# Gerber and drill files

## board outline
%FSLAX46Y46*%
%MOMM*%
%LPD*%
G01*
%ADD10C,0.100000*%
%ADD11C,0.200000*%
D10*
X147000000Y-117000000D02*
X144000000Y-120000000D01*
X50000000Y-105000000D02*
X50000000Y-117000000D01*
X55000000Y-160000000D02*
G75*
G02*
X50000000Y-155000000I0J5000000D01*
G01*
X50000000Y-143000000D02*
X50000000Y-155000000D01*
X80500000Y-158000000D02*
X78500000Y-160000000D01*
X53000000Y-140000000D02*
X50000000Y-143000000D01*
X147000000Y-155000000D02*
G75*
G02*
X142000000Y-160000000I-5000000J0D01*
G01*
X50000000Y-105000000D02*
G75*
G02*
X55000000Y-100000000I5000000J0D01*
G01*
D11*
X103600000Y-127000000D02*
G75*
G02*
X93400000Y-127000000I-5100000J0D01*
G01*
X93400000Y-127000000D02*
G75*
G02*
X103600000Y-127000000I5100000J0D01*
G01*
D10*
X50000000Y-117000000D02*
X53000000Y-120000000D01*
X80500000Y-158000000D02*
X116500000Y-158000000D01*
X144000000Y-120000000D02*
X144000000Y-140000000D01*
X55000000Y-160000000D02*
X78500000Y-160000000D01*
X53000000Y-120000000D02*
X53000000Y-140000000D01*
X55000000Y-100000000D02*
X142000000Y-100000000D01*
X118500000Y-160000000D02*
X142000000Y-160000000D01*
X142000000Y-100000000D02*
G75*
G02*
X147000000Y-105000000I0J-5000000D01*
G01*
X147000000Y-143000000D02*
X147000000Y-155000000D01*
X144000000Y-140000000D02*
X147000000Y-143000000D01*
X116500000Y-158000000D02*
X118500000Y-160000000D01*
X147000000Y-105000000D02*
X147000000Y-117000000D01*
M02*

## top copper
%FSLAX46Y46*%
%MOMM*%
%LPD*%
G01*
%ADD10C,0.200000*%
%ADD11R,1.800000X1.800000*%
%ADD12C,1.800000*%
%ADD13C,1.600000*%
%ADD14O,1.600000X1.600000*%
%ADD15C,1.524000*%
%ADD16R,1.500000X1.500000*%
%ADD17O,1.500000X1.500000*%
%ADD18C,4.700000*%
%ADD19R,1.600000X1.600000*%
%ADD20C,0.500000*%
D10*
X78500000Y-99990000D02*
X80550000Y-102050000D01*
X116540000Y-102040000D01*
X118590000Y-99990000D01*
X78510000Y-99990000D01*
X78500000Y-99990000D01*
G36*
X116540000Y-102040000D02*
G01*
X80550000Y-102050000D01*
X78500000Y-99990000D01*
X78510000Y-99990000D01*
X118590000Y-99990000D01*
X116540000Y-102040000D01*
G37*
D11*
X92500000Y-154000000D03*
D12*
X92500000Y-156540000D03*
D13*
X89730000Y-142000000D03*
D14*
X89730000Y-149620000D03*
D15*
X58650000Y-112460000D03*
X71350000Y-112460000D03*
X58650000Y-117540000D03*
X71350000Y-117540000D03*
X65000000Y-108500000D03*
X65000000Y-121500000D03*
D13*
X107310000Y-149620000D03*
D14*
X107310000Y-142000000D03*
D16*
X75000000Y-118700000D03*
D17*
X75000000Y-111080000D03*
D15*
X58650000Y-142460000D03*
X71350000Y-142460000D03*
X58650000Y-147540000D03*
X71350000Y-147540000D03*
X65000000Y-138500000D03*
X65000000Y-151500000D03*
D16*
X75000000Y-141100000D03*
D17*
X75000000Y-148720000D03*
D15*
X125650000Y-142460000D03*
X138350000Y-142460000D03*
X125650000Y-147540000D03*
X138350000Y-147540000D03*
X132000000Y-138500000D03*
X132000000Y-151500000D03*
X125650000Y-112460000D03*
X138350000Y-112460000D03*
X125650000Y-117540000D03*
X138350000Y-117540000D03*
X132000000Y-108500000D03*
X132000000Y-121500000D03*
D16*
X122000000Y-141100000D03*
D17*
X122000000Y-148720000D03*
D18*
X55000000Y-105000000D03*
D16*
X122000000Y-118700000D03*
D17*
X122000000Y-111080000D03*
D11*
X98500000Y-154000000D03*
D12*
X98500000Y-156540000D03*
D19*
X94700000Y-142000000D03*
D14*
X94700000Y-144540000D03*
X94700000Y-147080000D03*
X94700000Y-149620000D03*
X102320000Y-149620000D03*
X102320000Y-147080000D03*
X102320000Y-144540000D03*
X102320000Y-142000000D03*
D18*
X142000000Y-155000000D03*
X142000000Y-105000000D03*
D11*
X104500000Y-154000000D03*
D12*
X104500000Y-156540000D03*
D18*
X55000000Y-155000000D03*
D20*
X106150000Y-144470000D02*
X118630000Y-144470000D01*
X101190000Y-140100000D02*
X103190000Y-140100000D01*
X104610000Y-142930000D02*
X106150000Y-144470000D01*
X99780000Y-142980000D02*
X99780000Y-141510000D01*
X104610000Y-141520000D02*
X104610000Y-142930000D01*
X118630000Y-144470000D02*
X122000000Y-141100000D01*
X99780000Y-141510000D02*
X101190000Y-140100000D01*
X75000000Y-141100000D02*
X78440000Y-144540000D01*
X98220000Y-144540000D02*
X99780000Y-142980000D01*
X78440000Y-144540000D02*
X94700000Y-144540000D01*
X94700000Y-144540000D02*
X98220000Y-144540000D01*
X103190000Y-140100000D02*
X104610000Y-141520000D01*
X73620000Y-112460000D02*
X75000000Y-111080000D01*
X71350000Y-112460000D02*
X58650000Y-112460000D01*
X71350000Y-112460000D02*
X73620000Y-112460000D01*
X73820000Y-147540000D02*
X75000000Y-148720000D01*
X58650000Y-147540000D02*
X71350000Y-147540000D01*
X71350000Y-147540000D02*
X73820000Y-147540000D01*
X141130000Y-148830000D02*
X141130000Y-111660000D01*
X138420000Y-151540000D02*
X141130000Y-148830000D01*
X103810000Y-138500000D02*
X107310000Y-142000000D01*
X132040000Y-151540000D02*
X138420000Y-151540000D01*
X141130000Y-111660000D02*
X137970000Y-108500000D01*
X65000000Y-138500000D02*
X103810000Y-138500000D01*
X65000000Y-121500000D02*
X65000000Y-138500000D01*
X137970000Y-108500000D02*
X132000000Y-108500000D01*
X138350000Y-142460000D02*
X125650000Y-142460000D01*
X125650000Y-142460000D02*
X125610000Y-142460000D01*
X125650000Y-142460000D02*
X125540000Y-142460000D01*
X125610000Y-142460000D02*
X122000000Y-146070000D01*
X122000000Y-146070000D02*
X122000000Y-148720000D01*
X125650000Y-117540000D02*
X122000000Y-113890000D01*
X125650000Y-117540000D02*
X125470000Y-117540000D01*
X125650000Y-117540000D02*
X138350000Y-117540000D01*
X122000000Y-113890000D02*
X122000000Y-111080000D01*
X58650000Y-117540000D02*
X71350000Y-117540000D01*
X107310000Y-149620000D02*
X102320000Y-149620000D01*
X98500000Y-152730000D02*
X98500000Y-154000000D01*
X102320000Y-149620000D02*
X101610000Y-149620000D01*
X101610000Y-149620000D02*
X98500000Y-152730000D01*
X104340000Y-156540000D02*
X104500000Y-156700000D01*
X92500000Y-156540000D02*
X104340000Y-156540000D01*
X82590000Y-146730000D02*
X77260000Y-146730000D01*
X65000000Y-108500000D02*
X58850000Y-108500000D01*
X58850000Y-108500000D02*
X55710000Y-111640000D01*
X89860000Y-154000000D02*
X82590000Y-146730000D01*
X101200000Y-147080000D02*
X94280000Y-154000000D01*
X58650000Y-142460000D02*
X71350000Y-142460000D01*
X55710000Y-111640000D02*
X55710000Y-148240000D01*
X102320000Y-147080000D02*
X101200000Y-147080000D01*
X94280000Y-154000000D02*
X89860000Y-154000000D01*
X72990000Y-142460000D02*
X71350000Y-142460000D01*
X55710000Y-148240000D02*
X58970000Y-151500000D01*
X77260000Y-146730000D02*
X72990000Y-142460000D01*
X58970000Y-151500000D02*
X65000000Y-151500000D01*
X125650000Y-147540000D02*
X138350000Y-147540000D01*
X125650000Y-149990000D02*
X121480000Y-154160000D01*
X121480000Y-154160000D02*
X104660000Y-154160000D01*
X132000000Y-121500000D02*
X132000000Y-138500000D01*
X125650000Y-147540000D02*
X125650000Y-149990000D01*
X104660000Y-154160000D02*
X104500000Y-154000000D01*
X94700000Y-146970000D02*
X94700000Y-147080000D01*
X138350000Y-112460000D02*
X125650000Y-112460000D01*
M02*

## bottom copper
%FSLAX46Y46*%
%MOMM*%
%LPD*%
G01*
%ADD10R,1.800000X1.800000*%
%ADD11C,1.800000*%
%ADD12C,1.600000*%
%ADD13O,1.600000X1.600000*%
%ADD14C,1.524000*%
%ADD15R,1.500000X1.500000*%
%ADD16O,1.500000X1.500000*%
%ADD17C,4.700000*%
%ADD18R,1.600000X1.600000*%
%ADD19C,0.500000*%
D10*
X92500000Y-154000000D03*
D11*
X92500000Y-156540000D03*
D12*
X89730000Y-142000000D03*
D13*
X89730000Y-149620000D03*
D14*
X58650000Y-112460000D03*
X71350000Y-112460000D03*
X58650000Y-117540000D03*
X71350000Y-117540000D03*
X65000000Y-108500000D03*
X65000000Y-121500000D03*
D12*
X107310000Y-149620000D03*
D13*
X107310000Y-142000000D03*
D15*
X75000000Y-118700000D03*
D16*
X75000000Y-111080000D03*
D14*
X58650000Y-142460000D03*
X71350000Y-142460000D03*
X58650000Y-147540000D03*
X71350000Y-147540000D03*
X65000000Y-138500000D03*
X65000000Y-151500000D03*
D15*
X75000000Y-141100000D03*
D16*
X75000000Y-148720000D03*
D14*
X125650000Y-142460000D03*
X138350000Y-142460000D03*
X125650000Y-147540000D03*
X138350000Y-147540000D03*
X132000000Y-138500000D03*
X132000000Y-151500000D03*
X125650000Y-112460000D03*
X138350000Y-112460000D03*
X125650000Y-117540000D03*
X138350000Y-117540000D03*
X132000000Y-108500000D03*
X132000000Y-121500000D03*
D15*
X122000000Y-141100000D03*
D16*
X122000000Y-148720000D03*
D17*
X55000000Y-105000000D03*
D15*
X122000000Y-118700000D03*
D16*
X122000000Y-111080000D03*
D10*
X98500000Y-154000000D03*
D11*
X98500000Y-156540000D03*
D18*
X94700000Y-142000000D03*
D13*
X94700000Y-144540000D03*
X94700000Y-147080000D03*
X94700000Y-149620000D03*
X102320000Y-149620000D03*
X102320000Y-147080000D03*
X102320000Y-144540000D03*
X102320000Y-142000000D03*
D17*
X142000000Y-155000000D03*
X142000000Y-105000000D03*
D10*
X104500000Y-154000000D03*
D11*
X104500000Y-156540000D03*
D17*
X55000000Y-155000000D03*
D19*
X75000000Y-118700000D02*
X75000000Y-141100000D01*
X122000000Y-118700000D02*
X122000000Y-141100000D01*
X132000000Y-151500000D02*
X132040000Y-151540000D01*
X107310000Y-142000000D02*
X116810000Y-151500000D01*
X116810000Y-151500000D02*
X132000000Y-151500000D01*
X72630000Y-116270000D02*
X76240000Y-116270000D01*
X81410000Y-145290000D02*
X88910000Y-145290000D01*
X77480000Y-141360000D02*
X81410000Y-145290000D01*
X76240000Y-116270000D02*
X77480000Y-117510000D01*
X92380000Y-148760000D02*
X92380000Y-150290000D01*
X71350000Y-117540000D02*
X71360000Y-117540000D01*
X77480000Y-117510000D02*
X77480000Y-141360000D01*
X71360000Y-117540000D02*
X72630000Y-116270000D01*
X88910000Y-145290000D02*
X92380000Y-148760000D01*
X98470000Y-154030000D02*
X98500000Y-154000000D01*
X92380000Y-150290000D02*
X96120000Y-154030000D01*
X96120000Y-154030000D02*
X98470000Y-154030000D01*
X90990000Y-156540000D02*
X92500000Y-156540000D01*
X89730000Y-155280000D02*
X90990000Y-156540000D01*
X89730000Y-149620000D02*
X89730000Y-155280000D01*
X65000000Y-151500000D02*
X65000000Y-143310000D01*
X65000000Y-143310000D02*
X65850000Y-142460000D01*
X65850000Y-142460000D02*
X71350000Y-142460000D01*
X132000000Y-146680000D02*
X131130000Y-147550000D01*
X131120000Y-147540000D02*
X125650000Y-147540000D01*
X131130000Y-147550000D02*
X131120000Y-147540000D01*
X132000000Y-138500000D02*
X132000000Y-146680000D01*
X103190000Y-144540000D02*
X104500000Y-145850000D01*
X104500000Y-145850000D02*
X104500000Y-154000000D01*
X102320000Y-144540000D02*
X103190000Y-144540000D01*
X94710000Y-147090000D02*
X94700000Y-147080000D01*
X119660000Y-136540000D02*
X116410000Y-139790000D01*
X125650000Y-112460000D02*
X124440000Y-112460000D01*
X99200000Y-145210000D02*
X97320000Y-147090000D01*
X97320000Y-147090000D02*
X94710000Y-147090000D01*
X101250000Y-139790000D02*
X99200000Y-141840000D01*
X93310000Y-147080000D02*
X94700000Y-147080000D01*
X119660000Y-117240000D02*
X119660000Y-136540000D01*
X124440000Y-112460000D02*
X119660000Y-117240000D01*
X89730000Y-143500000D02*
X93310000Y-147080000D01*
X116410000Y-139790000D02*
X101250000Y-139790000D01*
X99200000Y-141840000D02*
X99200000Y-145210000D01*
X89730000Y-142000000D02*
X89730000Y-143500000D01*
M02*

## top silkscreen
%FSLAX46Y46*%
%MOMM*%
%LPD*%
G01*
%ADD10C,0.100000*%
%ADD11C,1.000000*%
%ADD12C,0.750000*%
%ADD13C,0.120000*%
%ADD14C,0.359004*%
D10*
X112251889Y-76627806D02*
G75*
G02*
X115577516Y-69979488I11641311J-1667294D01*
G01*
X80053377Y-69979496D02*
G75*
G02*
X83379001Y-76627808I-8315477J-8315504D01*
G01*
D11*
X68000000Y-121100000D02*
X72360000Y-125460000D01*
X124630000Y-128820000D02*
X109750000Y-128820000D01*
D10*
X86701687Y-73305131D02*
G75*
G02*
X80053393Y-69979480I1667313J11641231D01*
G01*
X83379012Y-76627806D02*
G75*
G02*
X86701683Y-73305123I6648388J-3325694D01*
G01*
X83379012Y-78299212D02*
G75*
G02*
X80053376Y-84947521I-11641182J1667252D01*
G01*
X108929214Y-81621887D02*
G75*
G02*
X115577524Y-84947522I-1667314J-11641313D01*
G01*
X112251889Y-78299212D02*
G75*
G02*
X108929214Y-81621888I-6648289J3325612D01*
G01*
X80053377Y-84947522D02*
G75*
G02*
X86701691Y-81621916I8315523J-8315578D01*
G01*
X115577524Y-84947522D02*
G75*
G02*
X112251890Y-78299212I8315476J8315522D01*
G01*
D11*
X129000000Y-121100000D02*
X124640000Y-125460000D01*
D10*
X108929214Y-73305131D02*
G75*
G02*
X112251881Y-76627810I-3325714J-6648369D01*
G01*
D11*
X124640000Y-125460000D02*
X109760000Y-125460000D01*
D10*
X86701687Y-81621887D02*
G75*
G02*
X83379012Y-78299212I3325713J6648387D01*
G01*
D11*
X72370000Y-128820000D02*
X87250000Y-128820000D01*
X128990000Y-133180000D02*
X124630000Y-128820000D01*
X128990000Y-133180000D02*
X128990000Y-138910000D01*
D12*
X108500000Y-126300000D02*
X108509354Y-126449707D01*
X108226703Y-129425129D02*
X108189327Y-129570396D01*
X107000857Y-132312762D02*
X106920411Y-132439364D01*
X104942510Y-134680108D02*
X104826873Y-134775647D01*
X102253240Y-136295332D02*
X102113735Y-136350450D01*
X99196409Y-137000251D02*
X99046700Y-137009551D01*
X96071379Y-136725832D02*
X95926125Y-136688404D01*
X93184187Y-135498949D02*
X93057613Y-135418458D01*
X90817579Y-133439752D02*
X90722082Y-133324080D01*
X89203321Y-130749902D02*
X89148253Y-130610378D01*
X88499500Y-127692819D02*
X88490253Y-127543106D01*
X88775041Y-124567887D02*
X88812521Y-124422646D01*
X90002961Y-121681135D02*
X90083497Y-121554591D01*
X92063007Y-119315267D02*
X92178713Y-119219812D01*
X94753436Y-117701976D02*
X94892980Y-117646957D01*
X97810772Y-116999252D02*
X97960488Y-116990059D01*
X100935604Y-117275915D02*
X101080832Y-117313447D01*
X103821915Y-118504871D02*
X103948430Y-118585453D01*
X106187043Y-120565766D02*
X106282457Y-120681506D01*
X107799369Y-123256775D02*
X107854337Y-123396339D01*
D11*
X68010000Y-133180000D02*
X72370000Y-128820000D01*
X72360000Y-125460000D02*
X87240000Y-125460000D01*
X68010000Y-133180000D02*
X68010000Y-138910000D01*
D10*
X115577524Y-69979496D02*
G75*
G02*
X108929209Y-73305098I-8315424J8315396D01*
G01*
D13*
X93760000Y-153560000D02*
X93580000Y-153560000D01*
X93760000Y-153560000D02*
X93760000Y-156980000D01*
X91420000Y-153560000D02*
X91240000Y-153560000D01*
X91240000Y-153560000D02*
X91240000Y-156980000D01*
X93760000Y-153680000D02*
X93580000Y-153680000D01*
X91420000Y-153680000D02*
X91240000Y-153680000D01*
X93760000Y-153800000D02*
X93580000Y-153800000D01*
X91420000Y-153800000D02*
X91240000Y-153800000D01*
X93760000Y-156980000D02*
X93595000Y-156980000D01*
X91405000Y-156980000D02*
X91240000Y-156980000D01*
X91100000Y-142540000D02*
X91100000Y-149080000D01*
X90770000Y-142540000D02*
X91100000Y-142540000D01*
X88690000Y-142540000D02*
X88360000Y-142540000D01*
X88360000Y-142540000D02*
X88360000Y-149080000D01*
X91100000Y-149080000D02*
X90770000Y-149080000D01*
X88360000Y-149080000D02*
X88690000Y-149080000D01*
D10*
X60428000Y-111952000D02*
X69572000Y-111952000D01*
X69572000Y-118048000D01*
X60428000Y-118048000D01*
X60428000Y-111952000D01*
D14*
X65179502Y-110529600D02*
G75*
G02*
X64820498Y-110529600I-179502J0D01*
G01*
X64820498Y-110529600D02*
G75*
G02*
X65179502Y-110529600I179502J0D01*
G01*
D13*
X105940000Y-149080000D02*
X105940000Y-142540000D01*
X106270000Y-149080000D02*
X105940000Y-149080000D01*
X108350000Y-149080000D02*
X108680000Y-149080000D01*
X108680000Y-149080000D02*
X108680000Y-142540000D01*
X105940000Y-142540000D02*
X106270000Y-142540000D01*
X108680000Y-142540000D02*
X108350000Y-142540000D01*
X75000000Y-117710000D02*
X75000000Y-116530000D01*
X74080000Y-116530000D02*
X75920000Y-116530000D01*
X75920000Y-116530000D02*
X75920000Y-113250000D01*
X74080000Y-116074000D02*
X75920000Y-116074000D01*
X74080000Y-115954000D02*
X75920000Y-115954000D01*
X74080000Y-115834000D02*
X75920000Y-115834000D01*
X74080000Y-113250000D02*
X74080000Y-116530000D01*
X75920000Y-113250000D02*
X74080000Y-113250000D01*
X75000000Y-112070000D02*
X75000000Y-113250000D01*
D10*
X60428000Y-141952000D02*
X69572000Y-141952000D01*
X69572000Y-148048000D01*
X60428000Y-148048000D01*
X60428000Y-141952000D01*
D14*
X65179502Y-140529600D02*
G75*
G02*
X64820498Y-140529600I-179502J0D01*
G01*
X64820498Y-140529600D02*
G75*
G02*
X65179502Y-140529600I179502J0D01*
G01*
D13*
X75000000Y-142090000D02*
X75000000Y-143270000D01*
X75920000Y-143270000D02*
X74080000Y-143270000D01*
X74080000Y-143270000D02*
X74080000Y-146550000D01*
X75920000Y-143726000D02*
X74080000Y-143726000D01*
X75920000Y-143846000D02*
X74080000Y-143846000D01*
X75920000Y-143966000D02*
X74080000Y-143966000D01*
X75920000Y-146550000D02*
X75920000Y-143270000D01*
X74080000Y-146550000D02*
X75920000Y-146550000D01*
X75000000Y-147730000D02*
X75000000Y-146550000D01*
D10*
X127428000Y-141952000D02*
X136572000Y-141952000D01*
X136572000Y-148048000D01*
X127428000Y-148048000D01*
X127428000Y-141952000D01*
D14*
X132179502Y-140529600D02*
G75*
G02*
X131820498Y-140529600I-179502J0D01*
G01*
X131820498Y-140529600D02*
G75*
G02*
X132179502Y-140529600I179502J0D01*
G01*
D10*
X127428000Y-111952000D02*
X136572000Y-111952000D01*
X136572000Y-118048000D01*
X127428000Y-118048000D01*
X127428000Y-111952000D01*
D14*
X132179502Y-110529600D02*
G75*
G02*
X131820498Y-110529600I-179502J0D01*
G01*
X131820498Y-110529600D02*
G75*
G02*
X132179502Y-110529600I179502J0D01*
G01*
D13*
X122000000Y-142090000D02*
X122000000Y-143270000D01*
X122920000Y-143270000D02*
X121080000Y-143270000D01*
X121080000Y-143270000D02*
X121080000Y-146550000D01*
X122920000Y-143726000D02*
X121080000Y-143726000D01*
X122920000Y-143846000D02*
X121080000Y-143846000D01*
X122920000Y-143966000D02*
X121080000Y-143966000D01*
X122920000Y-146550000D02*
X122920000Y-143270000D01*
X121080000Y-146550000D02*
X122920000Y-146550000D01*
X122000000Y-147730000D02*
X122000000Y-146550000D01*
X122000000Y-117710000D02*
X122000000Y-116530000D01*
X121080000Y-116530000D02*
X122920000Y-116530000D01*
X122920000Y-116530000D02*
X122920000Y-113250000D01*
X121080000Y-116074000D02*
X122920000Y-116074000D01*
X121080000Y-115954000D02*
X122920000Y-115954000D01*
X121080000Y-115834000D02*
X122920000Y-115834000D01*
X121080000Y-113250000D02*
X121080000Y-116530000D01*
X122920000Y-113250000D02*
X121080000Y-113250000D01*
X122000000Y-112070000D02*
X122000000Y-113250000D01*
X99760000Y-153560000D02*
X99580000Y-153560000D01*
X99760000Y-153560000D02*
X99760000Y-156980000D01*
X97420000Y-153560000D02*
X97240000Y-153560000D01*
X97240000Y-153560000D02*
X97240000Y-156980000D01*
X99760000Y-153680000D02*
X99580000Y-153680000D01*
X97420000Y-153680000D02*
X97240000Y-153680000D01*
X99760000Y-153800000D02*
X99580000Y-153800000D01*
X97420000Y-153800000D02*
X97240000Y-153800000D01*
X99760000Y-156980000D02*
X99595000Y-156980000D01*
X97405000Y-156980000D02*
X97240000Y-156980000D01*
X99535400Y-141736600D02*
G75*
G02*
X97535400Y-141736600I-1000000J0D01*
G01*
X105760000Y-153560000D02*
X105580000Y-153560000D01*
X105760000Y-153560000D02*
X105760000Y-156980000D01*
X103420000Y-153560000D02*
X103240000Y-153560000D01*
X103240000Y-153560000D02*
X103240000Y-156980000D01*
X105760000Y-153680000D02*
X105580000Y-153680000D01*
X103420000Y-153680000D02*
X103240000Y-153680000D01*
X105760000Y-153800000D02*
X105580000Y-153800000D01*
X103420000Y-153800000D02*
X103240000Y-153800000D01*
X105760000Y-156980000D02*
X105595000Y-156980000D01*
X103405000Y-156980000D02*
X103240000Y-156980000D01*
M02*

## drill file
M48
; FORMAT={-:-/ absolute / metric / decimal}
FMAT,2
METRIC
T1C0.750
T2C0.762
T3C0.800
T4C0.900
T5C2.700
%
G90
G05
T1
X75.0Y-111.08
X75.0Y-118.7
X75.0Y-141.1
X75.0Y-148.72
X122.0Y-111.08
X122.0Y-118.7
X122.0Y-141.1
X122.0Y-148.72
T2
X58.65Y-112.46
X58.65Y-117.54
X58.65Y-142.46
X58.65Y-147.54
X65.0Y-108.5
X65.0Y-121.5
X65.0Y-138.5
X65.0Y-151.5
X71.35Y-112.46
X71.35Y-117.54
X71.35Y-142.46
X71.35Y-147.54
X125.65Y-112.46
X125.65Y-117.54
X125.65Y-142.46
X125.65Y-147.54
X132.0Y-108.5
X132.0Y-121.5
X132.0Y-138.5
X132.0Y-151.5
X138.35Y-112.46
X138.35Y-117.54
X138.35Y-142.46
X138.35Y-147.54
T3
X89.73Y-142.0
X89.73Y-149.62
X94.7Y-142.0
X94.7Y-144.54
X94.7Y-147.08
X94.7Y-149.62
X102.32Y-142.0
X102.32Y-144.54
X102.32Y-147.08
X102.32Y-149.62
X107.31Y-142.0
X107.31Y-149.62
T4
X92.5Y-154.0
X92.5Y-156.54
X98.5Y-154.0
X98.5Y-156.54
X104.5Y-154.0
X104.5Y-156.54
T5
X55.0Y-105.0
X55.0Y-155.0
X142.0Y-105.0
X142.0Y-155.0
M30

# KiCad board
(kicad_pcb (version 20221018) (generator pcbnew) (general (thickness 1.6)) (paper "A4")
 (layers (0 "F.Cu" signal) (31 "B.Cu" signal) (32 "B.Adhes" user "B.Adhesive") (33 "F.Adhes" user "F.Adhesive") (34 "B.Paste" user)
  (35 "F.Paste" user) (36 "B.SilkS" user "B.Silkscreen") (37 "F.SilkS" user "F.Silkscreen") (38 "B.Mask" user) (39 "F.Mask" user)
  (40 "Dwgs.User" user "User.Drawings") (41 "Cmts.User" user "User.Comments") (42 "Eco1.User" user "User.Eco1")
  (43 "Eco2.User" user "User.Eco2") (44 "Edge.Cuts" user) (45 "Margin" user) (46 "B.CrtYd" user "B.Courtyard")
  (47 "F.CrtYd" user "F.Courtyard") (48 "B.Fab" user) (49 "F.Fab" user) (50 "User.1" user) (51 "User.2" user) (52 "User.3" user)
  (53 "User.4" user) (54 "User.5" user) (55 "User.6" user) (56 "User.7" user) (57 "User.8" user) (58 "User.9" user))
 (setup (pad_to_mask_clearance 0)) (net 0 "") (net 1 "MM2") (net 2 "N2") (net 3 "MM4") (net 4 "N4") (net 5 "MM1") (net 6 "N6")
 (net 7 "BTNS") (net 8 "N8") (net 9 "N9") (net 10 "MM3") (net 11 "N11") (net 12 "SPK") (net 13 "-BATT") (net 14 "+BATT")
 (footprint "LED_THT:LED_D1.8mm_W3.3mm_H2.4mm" (layer "F.Cu") (at 92.5 154 -90)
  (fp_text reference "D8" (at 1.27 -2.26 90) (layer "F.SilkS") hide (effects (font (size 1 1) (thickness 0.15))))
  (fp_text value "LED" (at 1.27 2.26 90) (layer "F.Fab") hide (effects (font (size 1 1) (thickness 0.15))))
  (fp_line (start -0.44 -1.26) (end -0.44 -1.08) (stroke (width 0.12) (type solid)) (layer "F.SilkS"))
  (fp_line (start -0.44 -1.26) (end 2.98 -1.26) (stroke (width 0.12) (type solid)) (layer "F.SilkS"))
  (fp_line (start -0.44 1.08) (end -0.44 1.26) (stroke (width 0.12) (type solid)) (layer "F.SilkS"))
  (fp_line (start -0.44 1.26) (end 2.98 1.26) (stroke (width 0.12) (type solid)) (layer "F.SilkS"))
  (fp_line (start -0.32 -1.26) (end -0.32 -1.08) (stroke (width 0.12) (type solid)) (layer "F.SilkS"))
  (fp_line (start -0.32 1.08) (end -0.32 1.26) (stroke (width 0.12) (type solid)) (layer "F.SilkS"))
  (fp_line (start -0.2 -1.26) (end -0.2 -1.08) (stroke (width 0.12) (type solid)) (layer "F.SilkS"))
  (fp_line (start -0.2 1.08) (end -0.2 1.26) (stroke (width 0.12) (type solid)) (layer "F.SilkS"))
  (fp_line (start 2.98 -1.26) (end 2.98 -1.095) (stroke (width 0.12) (type solid)) (layer "F.SilkS"))
  (fp_line (start 2.98 1.095) (end 2.98 1.26) (stroke (width 0.12) (type solid)) (layer "F.SilkS"))
  (pad "1" thru_hole rect (at 0 0 270) (size 1.8 1.8) (drill 0.9) (layers "*.Cu" "*.Mask") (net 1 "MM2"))
  (pad "2" thru_hole circle (at 2.54 0 270) (size 1.8 1.8) (drill 0.9) (layers "*.Cu" "*.Mask") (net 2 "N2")))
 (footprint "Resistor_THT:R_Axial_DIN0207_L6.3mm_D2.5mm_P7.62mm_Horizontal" (layer "F.Cu") (at 89.73 142 -90)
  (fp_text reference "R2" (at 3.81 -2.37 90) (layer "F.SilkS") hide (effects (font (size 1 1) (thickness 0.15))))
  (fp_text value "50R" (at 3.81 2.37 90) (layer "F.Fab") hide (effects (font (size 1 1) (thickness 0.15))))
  (fp_line (start 0.54 -1.37) (end 7.08 -1.37) (stroke (width 0.12) (type solid)) (layer "F.SilkS"))
  (fp_line (start 0.54 -1.04) (end 0.54 -1.37) (stroke (width 0.12) (type solid)) (layer "F.SilkS"))
  (fp_line (start 0.54 1.04) (end 0.54 1.37) (stroke (width 0.12) (type solid)) (layer "F.SilkS"))
  (fp_line (start 0.54 1.37) (end 7.08 1.37) (stroke (width 0.12) (type solid)) (layer "F.SilkS"))
  (fp_line (start 7.08 -1.37) (end 7.08 -1.04) (stroke (width 0.12) (type solid)) (layer "F.SilkS"))
  (fp_line (start 7.08 1.37) (end 7.08 1.04) (stroke (width 0.12) (type solid)) (layer "F.SilkS"))
  (pad "1" thru_hole circle (at 0 0 270) (size 1.6 1.6) (drill 0.8) (layers "*.Cu" "*.Mask") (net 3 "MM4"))
  (pad "2" thru_hole oval (at 7.62 0 270) (size 1.6 1.6) (drill 0.8) (layers "*.Cu" "*.Mask") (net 2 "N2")))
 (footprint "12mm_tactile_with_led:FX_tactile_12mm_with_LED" (layer "F.Cu") (at 65 115)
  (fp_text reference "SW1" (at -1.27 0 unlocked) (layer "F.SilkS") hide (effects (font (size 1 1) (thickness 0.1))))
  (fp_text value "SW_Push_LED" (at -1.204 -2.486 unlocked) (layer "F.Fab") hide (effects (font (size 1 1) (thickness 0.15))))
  (fp_rect (start -4.572 -3.048) (end 4.572 3.048) (stroke (width 0.1) (type default)) (fill none) (layer "F.SilkS"))
  (fp_circle (center 0 -4.4704) (end 0.309004 -4.4704) (stroke (width 0.1) (type solid)) (fill solid) (layer "F.SilkS"))
  (pad "1" thru_hole circle (at -6.35 -2.54) (size 1.524 1.524) (drill 0.762) (layers "*.Cu" "*.Mask") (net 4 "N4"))
  (pad "1" thru_hole circle (at 6.35 -2.54) (size 1.524 1.524) (drill 0.762) (layers "*.Cu" "*.Mask") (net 4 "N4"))
  (pad "2" thru_hole circle (at -6.35 2.54) (size 1.524 1.524) (drill 0.762) (layers "*.Cu" "*.Mask") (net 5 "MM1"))
  (pad "2" thru_hole circle (at 6.35 2.54) (size 1.524 1.524) (drill 0.762) (layers "*.Cu" "*.Mask") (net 5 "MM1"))
  (pad "3" thru_hole circle (at 0 -6.5) (size 1.524 1.524) (drill 0.762) (layers "*.Cu" "*.Mask") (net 1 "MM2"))
  (pad "4" thru_hole circle (at 0 6.5) (size 1.524 1.524) (drill 0.762) (layers "*.Cu" "*.Mask") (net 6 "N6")))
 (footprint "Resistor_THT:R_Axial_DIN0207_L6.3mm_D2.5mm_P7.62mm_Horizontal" (layer "F.Cu") (at 107.31 149.62 90)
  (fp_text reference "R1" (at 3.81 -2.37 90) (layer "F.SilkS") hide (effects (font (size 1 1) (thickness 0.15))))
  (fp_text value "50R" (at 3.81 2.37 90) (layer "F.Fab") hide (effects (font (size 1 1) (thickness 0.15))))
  (fp_line (start 0.54 -1.37) (end 7.08 -1.37) (stroke (width 0.12) (type solid)) (layer "F.SilkS"))
  (fp_line (start 0.54 -1.04) (end 0.54 -1.37) (stroke (width 0.12) (type solid)) (layer "F.SilkS"))
  (fp_line (start 0.54 1.04) (end 0.54 1.37) (stroke (width 0.12) (type solid)) (layer "F.SilkS"))
  (fp_line (start 0.54 1.37) (end 7.08 1.37) (stroke (width 0.12) (type solid)) (layer "F.SilkS"))
  (fp_line (start 7.08 -1.37) (end 7.08 -1.04) (stroke (width 0.12) (type solid)) (layer "F.SilkS"))
  (fp_line (start 7.08 1.37) (end 7.08 1.04) (stroke (width 0.12) (type solid)) (layer "F.SilkS"))
  (pad "1" thru_hole circle (at 0 0 90) (size 1.6 1.6) (drill 0.8) (layers "*.Cu" "*.Mask") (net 5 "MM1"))
  (pad "2" thru_hole oval (at 7.62 0 90) (size 1.6 1.6) (drill 0.8) (layers "*.Cu" "*.Mask") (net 6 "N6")))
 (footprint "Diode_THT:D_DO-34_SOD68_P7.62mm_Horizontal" (layer "F.Cu") (at 75 118.7 90)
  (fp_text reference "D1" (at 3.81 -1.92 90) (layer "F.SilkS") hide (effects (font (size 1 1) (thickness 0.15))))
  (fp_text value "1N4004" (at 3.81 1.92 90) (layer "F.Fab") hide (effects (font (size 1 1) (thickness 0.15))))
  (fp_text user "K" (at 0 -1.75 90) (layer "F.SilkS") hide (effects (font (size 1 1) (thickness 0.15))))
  (fp_line (start 0.99 0) (end 2.17 0) (stroke (width 0.12) (type solid)) (layer "F.SilkS"))
  (fp_line (start 2.17 -0.92) (end 2.17 0.92) (stroke (width 0.12) (type solid)) (layer "F.SilkS"))
  (fp_line (start 2.17 0.92) (end 5.45 0.92) (stroke (width 0.12) (type solid)) (layer "F.SilkS"))
  (fp_line (start 2.626 -0.92) (end 2.626 0.92) (stroke (width 0.12) (type solid)) (layer "F.SilkS"))
  (fp_line (start 2.746 -0.92) (end 2.746 0.92) (stroke (width 0.12) (type solid)) (layer "F.SilkS"))
  (fp_line (start 2.866 -0.92) (end 2.866 0.92) (stroke (width 0.12) (type solid)) (layer "F.SilkS"))
  (fp_line (start 5.45 -0.92) (end 2.17 -0.92) (stroke (width 0.12) (type solid)) (layer "F.SilkS"))
  (fp_line (start 5.45 0.92) (end 5.45 -0.92) (stroke (width 0.12) (type solid)) (layer "F.SilkS"))
  (fp_line (start 6.63 0) (end 5.45 0) (stroke (width 0.12) (type solid)) (layer "F.SilkS"))
  (pad "1" thru_hole rect (at 0 0 90) (size 1.5 1.5) (drill 0.75) (layers "*.Cu" "*.Mask") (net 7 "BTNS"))
  (pad "2" thru_hole oval (at 7.62 0 90) (size 1.5 1.5) (drill 0.75) (layers "*.Cu" "*.Mask") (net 4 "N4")))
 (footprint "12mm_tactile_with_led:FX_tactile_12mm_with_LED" (layer "F.Cu") (at 65 145)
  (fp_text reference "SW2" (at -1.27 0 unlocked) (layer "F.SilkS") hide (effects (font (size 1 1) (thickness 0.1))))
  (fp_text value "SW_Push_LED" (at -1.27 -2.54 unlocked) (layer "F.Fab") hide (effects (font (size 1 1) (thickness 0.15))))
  (fp_rect (start -4.572 -3.048) (end 4.572 3.048) (stroke (width 0.1) (type default)) (fill none) (layer "F.SilkS"))
  (fp_circle (center 0 -4.4704) (end 0.309004 -4.4704) (stroke (width 0.1) (type solid)) (fill solid) (layer "F.SilkS"))
  (pad "1" thru_hole circle (at -6.35 -2.54) (size 1.524 1.524) (drill 0.762) (layers "*.Cu" "*.Mask") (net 1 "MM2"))
  (pad "1" thru_hole circle (at 6.35 -2.54) (size 1.524 1.524) (drill 0.762) (layers "*.Cu" "*.Mask") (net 1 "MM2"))
  (pad "2" thru_hole circle (at -6.35 2.54) (size 1.524 1.524) (drill 0.762) (layers "*.Cu" "*.Mask") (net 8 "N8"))
  (pad "2" thru_hole circle (at 6.35 2.54) (size 1.524 1.524) (drill 0.762) (layers "*.Cu" "*.Mask") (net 8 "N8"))
  (pad "3" thru_hole circle (at 0 -6.5) (size 1.524 1.524) (drill 0.762) (layers "*.Cu" "*.Mask") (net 6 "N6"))
  (pad "4" thru_hole circle (at 0 6.5) (size 1.524 1.524) (drill 0.762) (layers "*.Cu" "*.Mask") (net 1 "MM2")))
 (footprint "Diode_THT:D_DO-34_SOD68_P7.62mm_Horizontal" (layer "F.Cu") (at 75 141.1 -90)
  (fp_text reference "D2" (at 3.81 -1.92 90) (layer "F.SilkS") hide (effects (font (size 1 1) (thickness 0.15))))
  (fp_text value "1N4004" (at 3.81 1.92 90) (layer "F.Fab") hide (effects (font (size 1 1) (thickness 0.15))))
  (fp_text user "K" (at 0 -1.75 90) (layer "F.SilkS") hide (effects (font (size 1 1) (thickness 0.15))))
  (fp_line (start 0.99 0) (end 2.17 0) (stroke (width 0.12) (type solid)) (layer "F.SilkS"))
  (fp_line (start 2.17 -0.92) (end 2.17 0.92) (stroke (width 0.12) (type solid)) (layer "F.SilkS"))
  (fp_line (start 2.17 0.92) (end 5.45 0.92) (stroke (width 0.12) (type solid)) (layer "F.SilkS"))
  (fp_line (start 2.626 -0.92) (end 2.626 0.92) (stroke (width 0.12) (type solid)) (layer "F.SilkS"))
  (fp_line (start 2.746 -0.92) (end 2.746 0.92) (stroke (width 0.12) (type solid)) (layer "F.SilkS"))
  (fp_line (start 2.866 -0.92) (end 2.866 0.92) (stroke (width 0.12) (type solid)) (layer "F.SilkS"))
  (fp_line (start 5.45 -0.92) (end 2.17 -0.92) (stroke (width 0.12) (type solid)) (layer "F.SilkS"))
  (fp_line (start 5.45 0.92) (end 5.45 -0.92) (stroke (width 0.12) (type solid)) (layer "F.SilkS"))
  (fp_line (start 6.63 0) (end 5.45 0) (stroke (width 0.12) (type solid)) (layer "F.SilkS"))
  (pad "1" thru_hole rect (at 0 0 270) (size 1.5 1.5) (drill 0.75) (layers "*.Cu" "*.Mask") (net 7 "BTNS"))
  (pad "2" thru_hole oval (at 7.62 0 270) (size 1.5 1.5) (drill 0.75) (layers "*.Cu" "*.Mask") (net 8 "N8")))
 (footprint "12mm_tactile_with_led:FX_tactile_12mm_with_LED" (layer "F.Cu") (at 132 145)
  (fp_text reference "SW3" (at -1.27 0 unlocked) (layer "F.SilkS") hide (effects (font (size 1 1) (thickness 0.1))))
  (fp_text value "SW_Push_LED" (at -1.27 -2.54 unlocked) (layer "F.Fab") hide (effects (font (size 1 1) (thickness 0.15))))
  (fp_rect (start -4.572 -3.048) (end 4.572 3.048) (stroke (width 0.1) (type default)) (fill none) (layer "F.SilkS"))
  (fp_circle (center 0 -4.4704) (end 0.309004 -4.4704) (stroke (width 0.1) (type solid)) (fill solid) (layer "F.SilkS"))
  (pad "1" thru_hole circle (at -6.35 -2.54) (size 1.524 1.524) (drill 0.762) (layers "*.Cu" "*.Mask") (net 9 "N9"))
  (pad "1" thru_hole circle (at 6.35 -2.54) (size 1.524 1.524) (drill 0.762) (layers "*.Cu" "*.Mask") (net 9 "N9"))
  (pad "2" thru_hole circle (at -6.35 2.54) (size 1.524 1.524) (drill 0.762) (layers "*.Cu" "*.Mask") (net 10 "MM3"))
  (pad "2" thru_hole circle (at 6.35 2.54) (size 1.524 1.524) (drill 0.762) (layers "*.Cu" "*.Mask") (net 10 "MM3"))
  (pad "3" thru_hole circle (at 0 -6.5) (size 1.524 1.524) (drill 0.762) (layers "*.Cu" "*.Mask") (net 10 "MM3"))
  (pad "4" thru_hole circle (at 0 6.5) (size 1.524 1.524) (drill 0.762) (layers "*.Cu" "*.Mask") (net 6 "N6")))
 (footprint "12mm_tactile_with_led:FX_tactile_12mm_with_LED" (layer "F.Cu") (at 132 115)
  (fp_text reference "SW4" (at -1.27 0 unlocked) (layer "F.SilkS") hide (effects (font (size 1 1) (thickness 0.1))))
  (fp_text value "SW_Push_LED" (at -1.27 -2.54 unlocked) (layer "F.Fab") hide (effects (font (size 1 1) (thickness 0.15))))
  (fp_rect (start -4.572 -3.048) (end 4.572 3.048) (stroke (width 0.1) (type default)) (fill none) (layer "F.SilkS"))
  (fp_circle (center 0 -4.4704) (end 0.309004 -4.4704) (stroke (width 0.1) (type solid)) (fill solid) (layer "F.SilkS"))
  (pad "1" thru_hole circle (at -6.35 -2.54) (size 1.524 1.524) (drill 0.762) (layers "*.Cu" "*.Mask") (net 3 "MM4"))
  (pad "1" thru_hole circle (at 6.35 -2.54) (size 1.524 1.524) (drill 0.762) (layers "*.Cu" "*.Mask") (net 3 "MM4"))
  (pad "2" thru_hole circle (at -6.35 2.54) (size 1.524 1.524) (drill 0.762) (layers "*.Cu" "*.Mask") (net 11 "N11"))
  (pad "2" thru_hole circle (at 6.35 2.54) (size 1.524 1.524) (drill 0.762) (layers "*.Cu" "*.Mask") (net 11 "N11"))
  (pad "3" thru_hole circle (at 0 -6.5) (size 1.524 1.524) (drill 0.762) (layers "*.Cu" "*.Mask") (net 6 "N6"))
  (pad "4" thru_hole circle (at 0 6.5) (size 1.524 1.524) (drill 0.762) (layers "*.Cu" "*.Mask") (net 10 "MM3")))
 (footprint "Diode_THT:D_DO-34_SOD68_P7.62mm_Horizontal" (layer "F.Cu") (at 122 141.1 -90)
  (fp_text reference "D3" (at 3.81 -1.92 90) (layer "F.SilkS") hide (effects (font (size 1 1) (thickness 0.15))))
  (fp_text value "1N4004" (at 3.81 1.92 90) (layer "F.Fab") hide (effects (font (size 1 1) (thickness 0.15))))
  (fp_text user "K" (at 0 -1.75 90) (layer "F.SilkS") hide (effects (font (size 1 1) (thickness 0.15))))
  (fp_line (start 0.99 0) (end 2.17 0) (stroke (width 0.12) (type solid)) (layer "F.SilkS"))
  (fp_line (start 2.17 -0.92) (end 2.17 0.92) (stroke (width 0.12) (type solid)) (layer "F.SilkS"))
  (fp_line (start 2.17 0.92) (end 5.45 0.92) (stroke (width 0.12) (type solid)) (layer "F.SilkS"))
  (fp_line (start 2.626 -0.92) (end 2.626 0.92) (stroke (width 0.12) (type solid)) (layer "F.SilkS"))
  (fp_line (start 2.746 -0.92) (end 2.746 0.92) (stroke (width 0.12) (type solid)) (layer "F.SilkS"))
  (fp_line (start 2.866 -0.92) (end 2.866 0.92) (stroke (width 0.12) (type solid)) (layer "F.SilkS"))
  (fp_line (start 5.45 -0.92) (end 2.17 -0.92) (stroke (width 0.12) (type solid)) (layer "F.SilkS"))
  (fp_line (start 5.45 0.92) (end 5.45 -0.92) (stroke (width 0.12) (type solid)) (layer "F.SilkS"))
  (fp_line (start 6.63 0) (end 5.45 0) (stroke (width 0.12) (type solid)) (layer "F.SilkS"))
  (pad "1" thru_hole rect (at 0 0 270) (size 1.5 1.5) (drill 0.75) (layers "*.Cu" "*.Mask") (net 7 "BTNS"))
  (pad "2" thru_hole oval (at 7.62 0 270) (size 1.5 1.5) (drill 0.75) (layers "*.Cu" "*.Mask") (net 9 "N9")))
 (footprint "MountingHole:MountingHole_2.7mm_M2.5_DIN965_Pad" (layer "F.Cu") (at 55 105)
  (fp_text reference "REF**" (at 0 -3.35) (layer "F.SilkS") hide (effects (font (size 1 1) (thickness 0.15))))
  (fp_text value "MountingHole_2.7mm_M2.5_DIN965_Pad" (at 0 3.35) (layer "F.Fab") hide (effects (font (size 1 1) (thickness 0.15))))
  (pad "1" thru_hole circle (at 0 0) (size 4.7 4.7) (drill 2.7) (layers "*.Cu" "*.Mask")))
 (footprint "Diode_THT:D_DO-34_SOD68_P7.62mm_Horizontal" (layer "F.Cu") (at 122 118.7 90)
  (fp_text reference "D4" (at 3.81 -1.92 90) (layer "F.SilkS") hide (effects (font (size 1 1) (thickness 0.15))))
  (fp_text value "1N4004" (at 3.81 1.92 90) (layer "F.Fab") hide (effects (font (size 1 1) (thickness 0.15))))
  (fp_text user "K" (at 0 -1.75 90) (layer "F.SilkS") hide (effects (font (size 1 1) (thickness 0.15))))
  (fp_line (start 0.99 0) (end 2.17 0) (stroke (width 0.12) (type solid)) (layer "F.SilkS"))
  (fp_line (start 2.17 -0.92) (end 2.17 0.92) (stroke (width 0.12) (type solid)) (layer "F.SilkS"))
  (fp_line (start 2.17 0.92) (end 5.45 0.92) (stroke (width 0.12) (type solid)) (layer "F.SilkS"))
  (fp_line (start 2.626 -0.92) (end 2.626 0.92) (stroke (width 0.12) (type solid)) (layer "F.SilkS"))
  (fp_line (start 2.746 -0.92) (end 2.746 0.92) (stroke (width 0.12) (type solid)) (layer "F.SilkS"))
  (fp_line (start 2.866 -0.92) (end 2.866 0.92) (stroke (width 0.12) (type solid)) (layer "F.SilkS"))
  (fp_line (start 5.45 -0.92) (end 2.17 -0.92) (stroke (width 0.12) (type solid)) (layer "F.SilkS"))
  (fp_line (start 5.45 0.92) (end 5.45 -0.92) (stroke (width 0.12) (type solid)) (layer "F.SilkS"))
  (fp_line (start 6.63 0) (end 5.45 0) (stroke (width 0.12) (type solid)) (layer "F.SilkS"))
  (pad "1" thru_hole rect (at 0 0 90) (size 1.5 1.5) (drill 0.75) (layers "*.Cu" "*.Mask") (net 7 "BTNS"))
  (pad "2" thru_hole oval (at 7.62 0 90) (size 1.5 1.5) (drill 0.75) (layers "*.Cu" "*.Mask") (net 11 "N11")))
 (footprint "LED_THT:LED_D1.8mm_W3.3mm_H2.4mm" (layer "F.Cu") (at 98.5 154 -90)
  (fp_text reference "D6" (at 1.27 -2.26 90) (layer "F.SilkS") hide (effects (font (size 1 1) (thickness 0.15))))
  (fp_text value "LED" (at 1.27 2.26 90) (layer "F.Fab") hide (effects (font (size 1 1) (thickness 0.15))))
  (fp_line (start -0.44 -1.26) (end -0.44 -1.08) (stroke (width 0.12) (type solid)) (layer "F.SilkS"))
  (fp_line (start -0.44 -1.26) (end 2.98 -1.26) (stroke (width 0.12) (type solid)) (layer "F.SilkS"))
  (fp_line (start -0.44 1.08) (end -0.44 1.26) (stroke (width 0.12) (type solid)) (layer "F.SilkS"))
  (fp_line (start -0.44 1.26) (end 2.98 1.26) (stroke (width 0.12) (type solid)) (layer "F.SilkS"))
  (fp_line (start -0.32 -1.26) (end -0.32 -1.08) (stroke (width 0.12) (type solid)) (layer "F.SilkS"))
  (fp_line (start -0.32 1.08) (end -0.32 1.26) (stroke (width 0.12) (type solid)) (layer "F.SilkS"))
  (fp_line (start -0.2 -1.26) (end -0.2 -1.08) (stroke (width 0.12) (type solid)) (layer "F.SilkS"))
  (fp_line (start -0.2 1.08) (end -0.2 1.26) (stroke (width 0.12) (type solid)) (layer "F.SilkS"))
  (fp_line (start 2.98 -1.26) (end 2.98 -1.095) (stroke (width 0.12) (type solid)) (layer "F.SilkS"))
  (fp_line (start 2.98 1.095) (end 2.98 1.26) (stroke (width 0.12) (type solid)) (layer "F.SilkS"))
  (pad "1" thru_hole rect (at 0 0 270) (size 1.8 1.8) (drill 0.9) (layers "*.Cu" "*.Mask") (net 5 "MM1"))
  (pad "2" thru_hole circle (at 2.54 0 270) (size 1.8 1.8) (drill 0.9) (layers "*.Cu" "*.Mask") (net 2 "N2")))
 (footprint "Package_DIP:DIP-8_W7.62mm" (layer "F.Cu") (at 94.7 142)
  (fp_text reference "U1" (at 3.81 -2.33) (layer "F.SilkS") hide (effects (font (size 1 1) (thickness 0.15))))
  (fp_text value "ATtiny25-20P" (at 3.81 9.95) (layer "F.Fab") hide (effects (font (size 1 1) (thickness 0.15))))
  (fp_arc (start 4.8354 -0.2634) (mid 3.8354 0.7366) (end 2.8354 -0.2634) (stroke (width 0.12) (type solid)) (layer "F.SilkS"))
  (pad "1" thru_hole rect (at 0 0) (size 1.6 1.6) (drill 0.8) (layers "*.Cu" "*.Mask") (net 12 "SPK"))
  (pad "2" thru_hole oval (at 0 2.54) (size 1.6 1.6) (drill 0.8) (layers "*.Cu" "*.Mask") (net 7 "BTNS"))
  (pad "3" thru_hole oval (at 0 5.08) (size 1.6 1.6) (drill 0.8) (layers "*.Cu" "*.Mask") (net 3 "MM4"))
  (pad "4" thru_hole oval (at 0 7.62) (size 1.6 1.6) (drill 0.8) (layers "*.Cu" "*.Mask") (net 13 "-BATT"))
  (pad "5" thru_hole oval (at 7.62 7.62) (size 1.6 1.6) (drill 0.8) (layers "*.Cu" "*.Mask") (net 5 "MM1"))
  (pad "6" thru_hole oval (at 7.62 5.08) (size 1.6 1.6) (drill 0.8) (layers "*.Cu" "*.Mask") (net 1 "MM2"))
  (pad "7" thru_hole oval (at 7.62 2.54) (size 1.6 1.6) (drill 0.8) (layers "*.Cu" "*.Mask") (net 10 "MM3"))
  (pad "8" thru_hole oval (at 7.62 0) (size 1.6 1.6) (drill 0.8) (layers "*.Cu" "*.Mask") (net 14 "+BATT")))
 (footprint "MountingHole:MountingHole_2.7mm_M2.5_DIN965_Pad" (layer "F.Cu") (at 142 155)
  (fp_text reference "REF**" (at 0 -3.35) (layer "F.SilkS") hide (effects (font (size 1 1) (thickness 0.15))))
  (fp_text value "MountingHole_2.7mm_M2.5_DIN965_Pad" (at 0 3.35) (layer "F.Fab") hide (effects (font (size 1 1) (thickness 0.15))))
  (pad "1" thru_hole circle (at 0 0) (size 4.7 4.7) (drill 2.7) (layers "*.Cu" "*.Mask")))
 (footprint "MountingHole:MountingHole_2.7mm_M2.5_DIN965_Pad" (layer "F.Cu") (at 142 105)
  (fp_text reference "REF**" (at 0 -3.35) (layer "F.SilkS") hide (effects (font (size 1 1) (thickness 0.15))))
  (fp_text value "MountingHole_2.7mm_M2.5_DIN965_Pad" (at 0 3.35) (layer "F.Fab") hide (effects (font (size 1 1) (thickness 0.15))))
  (pad "1" thru_hole circle (at 0 0) (size 4.7 4.7) (drill 2.7) (layers "*.Cu" "*.Mask")))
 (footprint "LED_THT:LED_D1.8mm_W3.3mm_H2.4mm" (layer "F.Cu") (at 104.5 154 -90)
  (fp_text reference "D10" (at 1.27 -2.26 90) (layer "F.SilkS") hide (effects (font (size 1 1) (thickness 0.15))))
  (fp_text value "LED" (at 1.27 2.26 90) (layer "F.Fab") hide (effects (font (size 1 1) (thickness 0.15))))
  (fp_line (start -0.44 -1.26) (end -0.44 -1.08) (stroke (width 0.12) (type solid)) (layer "F.SilkS"))
  (fp_line (start -0.44 -1.26) (end 2.98 -1.26) (stroke (width 0.12) (type solid)) (layer "F.SilkS"))
  (fp_line (start -0.44 1.08) (end -0.44 1.26) (stroke (width 0.12) (type solid)) (layer "F.SilkS"))
  (fp_line (start -0.44 1.26) (end 2.98 1.26) (stroke (width 0.12) (type solid)) (layer "F.SilkS"))
  (fp_line (start -0.32 -1.26) (end -0.32 -1.08) (stroke (width 0.12) (type solid)) (layer "F.SilkS"))
  (fp_line (start -0.32 1.08) (end -0.32 1.26) (stroke (width 0.12) (type solid)) (layer "F.SilkS"))
  (fp_line (start -0.2 -1.26) (end -0.2 -1.08) (stroke (width 0.12) (type solid)) (layer "F.SilkS"))
  (fp_line (start -0.2 1.08) (end -0.2 1.26) (stroke (width 0.12) (type solid)) (layer "F.SilkS"))
  (fp_line (start 2.98 -1.26) (end 2.98 -1.095) (stroke (width 0.12) (type solid)) (layer "F.SilkS"))
  (fp_line (start 2.98 1.095) (end 2.98 1.26) (stroke (width 0.12) (type solid)) (layer "F.SilkS"))
  (pad "1" thru_hole rect (at 0 0 270) (size 1.8 1.8) (drill 0.9) (layers "*.Cu" "*.Mask") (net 10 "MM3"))
  (pad "2" thru_hole circle (at 2.54 0 270) (size 1.8 1.8) (drill 0.9) (layers "*.Cu" "*.Mask") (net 2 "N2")))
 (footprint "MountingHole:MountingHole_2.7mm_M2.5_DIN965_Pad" (layer "F.Cu") (at 55 155)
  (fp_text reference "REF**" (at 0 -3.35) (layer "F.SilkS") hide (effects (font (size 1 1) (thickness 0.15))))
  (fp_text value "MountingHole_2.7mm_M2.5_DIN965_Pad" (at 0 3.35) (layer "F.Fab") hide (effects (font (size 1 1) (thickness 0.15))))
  (pad "1" thru_hole circle (at 0 0) (size 4.7 4.7) (drill 2.7) (layers "*.Cu" "*.Mask")))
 (gr_poly
  (pts (xy 78.5 99.99) (xy 80.55 102.05) (xy 116.54 102.04) (xy 118.59 99.99) (xy 78.51 99.99)) (stroke (width 0.2) (type solid))
  (fill solid) (layer "F.Cu"))
 (gr_arc (start 112.251889 76.627806) (mid 113.375579 73.033969) (end 115.577524 69.979496) (stroke (width 0.1) (type default))
  (layer "F.SilkS"))
 (gr_arc (start 80.053377 69.979496) (mid 82.255333 73.033963) (end 83.379012 76.627806) (stroke (width 0.1) (type default))
  (layer "F.SilkS"))
 (gr_line (start 68 121.1) (end 72.36 125.46) (stroke (width 1) (type default)) (layer "F.SilkS"))
 (gr_line (start 124.63 128.82) (end 109.75 128.82) (stroke (width 1) (type default)) (layer "F.SilkS"))
 (gr_arc (start 86.701687 73.305131) (mid 83.107847 72.181445) (end 80.053377 69.979496) (stroke (width 0.1) (type default))
  (layer "F.SilkS"))
 (gr_arc (start 83.379012 76.627806) (mid 84.770906 74.697025) (end 86.701687 73.305131) (stroke (width 0.1) (type default))
  (layer "F.SilkS"))
 (gr_arc (start 83.379012 78.299212) (mid 82.255328 81.893054) (end 80.053377 84.947522) (stroke (width 0.1) (type default))
  (layer "F.SilkS"))
 (gr_arc (start 108.929214 81.621887) (mid 112.523051 82.745578) (end 115.577524 84.947522) (stroke (width 0.1) (type default))
  (layer "F.SilkS"))
 (gr_arc (start 112.251889 78.299212) (mid 110.86 80.23) (end 108.929214 81.621887) (stroke (width 0.1) (type default)) (layer "F.SilkS"))
 (gr_arc (start 80.053377 84.947522) (mid 83.107845 82.74557) (end 86.701687 81.621887) (stroke (width 0.1) (type default))
  (layer "F.SilkS"))
 (gr_arc (start 115.577524 84.947522) (mid 113.375568 81.893056) (end 112.251889 78.299212) (stroke (width 0.1) (type default))
  (layer "F.SilkS"))
 (gr_line (start 129 121.1) (end 124.64 125.46) (stroke (width 1) (type default)) (layer "F.SilkS"))
 (gr_arc (start 108.929214 73.305131) (mid 110.859993 74.697026) (end 112.251889 76.627806) (stroke (width 0.1) (type default))
  (layer "F.SilkS"))
 (gr_line (start 124.64 125.46) (end 109.76 125.46) (stroke (width 1) (type default)) (layer "F.SilkS"))
 (gr_arc (start 86.701687 81.621887) (mid 84.770905 80.229994) (end 83.379012 78.299212) (stroke (width 0.1) (type default))
  (layer "F.SilkS"))
 (gr_line (start 72.37 128.82) (end 87.25 128.82) (stroke (width 1) (type default)) (layer "F.SilkS"))
 (gr_line (start 128.99 133.18) (end 124.63 128.82) (stroke (width 1) (type default)) (layer "F.SilkS"))
 (gr_line (start 128.99 133.18) (end 128.99 138.91) (stroke (width 1) (type default)) (layer "F.SilkS"))
 (gr_circle (center 98.5 127) (end 108.5 126.3) (stroke (width 0.75) (type dot)) (fill none) (layer "F.SilkS"))
 (gr_line (start 68.01 133.18) (end 72.37 128.82) (stroke (width 1) (type default)) (layer "F.SilkS"))
 (gr_line (start 72.36 125.46) (end 87.24 125.46) (stroke (width 1) (type default)) (layer "F.SilkS"))
 (gr_line (start 68.01 133.18) (end 68.01 138.91) (stroke (width 1) (type default)) (layer "F.SilkS"))
 (gr_arc (start 115.577524 69.979496) (mid 112.523059 72.181457) (end 108.929214 73.305131) (stroke (width 0.1) (type default))
  (layer "F.SilkS"))
 (gr_line (start 147 117) (end 144 120) (stroke (width 0.1) (type default)) (layer "Edge.Cuts"))
 (gr_line (start 50 105) (end 50 117) (stroke (width 0.1) (type default)) (layer "Edge.Cuts"))
 (gr_arc (start 55 160) (mid 51.464466 158.535534) (end 50 155) (stroke (width 0.1) (type default)) (layer "Edge.Cuts"))
 (gr_line (start 50 143) (end 50 155) (stroke (width 0.1) (type default)) (layer "Edge.Cuts"))
 (gr_line (start 80.5 158) (end 78.5 160) (stroke (width 0.1) (type default)) (layer "Edge.Cuts"))
 (gr_line (start 53 140) (end 50 143) (stroke (width 0.1) (type default)) (layer "Edge.Cuts"))
 (gr_arc (start 147 155) (mid 145.535534 158.535534) (end 142 160) (stroke (width 0.1) (type default)) (layer "Edge.Cuts"))
 (gr_arc (start 50 105) (mid 51.464466 101.464466) (end 55 100) (stroke (width 0.1) (type default)) (layer "Edge.Cuts"))
 (gr_circle (center 98.5 127) (end 103.6 127) (stroke (width 0.2) (type default)) (fill none) (layer "Edge.Cuts"))
 (gr_line (start 50 117) (end 53 120) (stroke (width 0.1) (type default)) (layer "Edge.Cuts"))
 (gr_line (start 80.5 158) (end 116.5 158) (stroke (width 0.1) (type default)) (layer "Edge.Cuts"))
 (gr_line (start 144 120) (end 144 140) (stroke (width 0.1) (type default)) (layer "Edge.Cuts"))
 (gr_line (start 55 160) (end 78.5 160) (stroke (width 0.1) (type default)) (layer "Edge.Cuts"))
 (gr_line (start 53 120) (end 53 140) (stroke (width 0.1) (type default)) (layer "Edge.Cuts"))
 (gr_line (start 55 100) (end 142 100) (stroke (width 0.1) (type default)) (layer "Edge.Cuts"))
 (gr_line (start 118.5 160) (end 142 160) (stroke (width 0.1) (type default)) (layer "Edge.Cuts"))
 (gr_arc (start 142 100) (mid 145.535534 101.464466) (end 147 105) (stroke (width 0.1) (type default)) (layer "Edge.Cuts"))
 (gr_line (start 147 143) (end 147 155) (stroke (width 0.1) (type default)) (layer "Edge.Cuts"))
 (gr_line (start 144 140) (end 147 143) (stroke (width 0.1) (type default)) (layer "Edge.Cuts"))
 (gr_line (start 116.5 158) (end 118.5 160) (stroke (width 0.1) (type default)) (layer "Edge.Cuts"))
 (gr_line (start 147 105) (end 147 117) (stroke (width 0.1) (type default)) (layer "Edge.Cuts"))
 (segment (start 106.15 144.47) (end 118.63 144.47) (width 0.5) (layer "F.Cu") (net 7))
 (segment (start 101.19 140.1) (end 103.19 140.1) (width 0.5) (layer "F.Cu") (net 7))
 (segment (start 104.61 142.93) (end 106.15 144.47) (width 0.5) (layer "F.Cu") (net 7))
 (segment (start 99.78 142.98) (end 99.78 141.51) (width 0.5) (layer "F.Cu") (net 7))
 (segment (start 104.61 141.52) (end 104.61 142.93) (width 0.5) (layer "F.Cu") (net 7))
 (segment (start 118.63 144.47) (end 122 141.1) (width 0.5) (layer "F.Cu") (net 7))
 (segment (start 99.78 141.51) (end 101.19 140.1) (width 0.5) (layer "F.Cu") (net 7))
 (segment (start 75 141.1) (end 78.44 144.54) (width 0.5) (layer "F.Cu") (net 7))
 (segment (start 98.22 144.54) (end 99.78 142.98) (width 0.5) (layer "F.Cu") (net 7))
 (segment (start 78.44 144.54) (end 94.7 144.54) (width 0.5) (layer "F.Cu") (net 7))
 (segment (start 94.7 144.54) (end 98.22 144.54) (width 0.5) (layer "F.Cu") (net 7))
 (segment (start 103.19 140.1) (end 104.61 141.52) (width 0.5) (layer "F.Cu") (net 7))
 (segment (start 75 118.7) (end 75 141.1) (width 0.5) (layer "B.Cu") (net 7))
 (segment (start 122 118.7) (end 122 141.1) (width 0.5) (layer "B.Cu") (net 7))
 (segment (start 73.62 112.46) (end 75 111.08) (width 0.5) (layer "F.Cu") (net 4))
 (segment (start 71.35 112.46) (end 58.65 112.46) (width 0.5) (layer "F.Cu") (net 4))
 (segment (start 71.35 112.46) (end 73.62 112.46) (width 0.5) (layer "F.Cu") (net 4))
 (segment (start 73.82 147.54) (end 75 148.72) (width 0.5) (layer "F.Cu") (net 8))
 (segment (start 58.65 147.54) (end 71.35 147.54) (width 0.5) (layer "F.Cu") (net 8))
 (segment (start 71.35 147.54) (end 73.82 147.54) (width 0.5) (layer "F.Cu") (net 8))
 (segment (start 141.13 148.83) (end 141.13 111.66) (width 0.5) (layer "F.Cu") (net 6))
 (segment (start 138.42 151.54) (end 141.13 148.83) (width 0.5) (layer "F.Cu") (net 6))
 (segment (start 103.81 138.5) (end 107.31 142) (width 0.5) (layer "F.Cu") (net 6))
 (segment (start 132.04 151.54) (end 138.42 151.54) (width 0.5) (layer "F.Cu") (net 6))
 (segment (start 141.13 111.66) (end 137.97 108.5) (width 0.5) (layer "F.Cu") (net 6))
 (segment (start 65 138.5) (end 103.81 138.5) (width 0.5) (layer "F.Cu") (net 6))
 (segment (start 65 121.5) (end 65 138.5) (width 0.5) (layer "F.Cu") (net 6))
 (segment (start 137.97 108.5) (end 132 108.5) (width 0.5) (layer "F.Cu") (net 6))
 (segment (start 132 151.5) (end 132.04 151.54) (width 0.5) (layer "B.Cu") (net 6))
 (segment (start 107.31 142) (end 116.81 151.5) (width 0.5) (layer "B.Cu") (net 6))
 (segment (start 116.81 151.5) (end 132 151.5) (width 0.5) (layer "B.Cu") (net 6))
 (segment (start 138.35 142.46) (end 125.65 142.46) (width 0.5) (layer "F.Cu") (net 9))
 (segment (start 125.65 142.46) (end 125.61 142.46) (width 0.5) (layer "F.Cu") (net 9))
 (segment (start 125.65 142.46) (end 125.54 142.46) (width 0.5) (layer "F.Cu") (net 9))
 (segment (start 125.61 142.46) (end 122 146.07) (width 0.5) (layer "F.Cu") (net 9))
 (segment (start 122 146.07) (end 122 148.72) (width 0.5) (layer "F.Cu") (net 9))
 (segment (start 125.65 117.54) (end 122 113.89) (width 0.5) (layer "F.Cu") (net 11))
 (segment (start 125.65 117.54) (end 125.47 117.54) (width 0.5) (layer "F.Cu") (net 11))
 (segment (start 125.65 117.54) (end 138.35 117.54) (width 0.5) (layer "F.Cu") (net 11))
 (segment (start 122 113.89) (end 122 111.08) (width 0.5) (layer "F.Cu") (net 11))
 (segment (start 58.65 117.54) (end 71.35 117.54) (width 0.5) (layer "F.Cu") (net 5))
 (segment (start 107.31 149.62) (end 102.32 149.62) (width 0.5) (layer "F.Cu") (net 5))
 (segment (start 98.5 152.73) (end 98.5 154) (width 0.5) (layer "F.Cu") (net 5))
 (segment (start 102.32 149.62) (end 101.61 149.62) (width 0.5) (layer "F.Cu") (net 5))
 (segment (start 101.61 149.62) (end 98.5 152.73) (width 0.5) (layer "F.Cu") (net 5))
 (segment (start 72.63 116.27) (end 76.24 116.27) (width 0.5) (layer "B.Cu") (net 5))
 (segment (start 81.41 145.29) (end 88.91 145.29) (width 0.5) (layer "B.Cu") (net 5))
 (segment (start 77.48 141.36) (end 81.41 145.29) (width 0.5) (layer "B.Cu") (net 5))
 (segment (start 76.24 116.27) (end 77.48 117.51) (width 0.5) (layer "B.Cu") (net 5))
 (segment (start 92.38 148.76) (end 92.38 150.29) (width 0.5) (layer "B.Cu") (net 5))
 (segment (start 71.35 117.54) (end 71.36 117.54) (width 0.5) (layer "B.Cu") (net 5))
 (segment (start 77.48 117.51) (end 77.48 141.36) (width 0.5) (layer "B.Cu") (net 5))
 (segment (start 71.36 117.54) (end 72.63 116.27) (width 0.5) (layer "B.Cu") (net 5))
 (segment (start 88.91 145.29) (end 92.38 148.76) (width 0.5) (layer "B.Cu") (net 5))
 (segment (start 98.47 154.03) (end 98.5 154) (width 0.5) (layer "B.Cu") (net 5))
 (segment (start 92.38 150.29) (end 96.12 154.03) (width 0.5) (layer "B.Cu") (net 5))
 (segment (start 96.12 154.03) (end 98.47 154.03) (width 0.5) (layer "B.Cu") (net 5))
 (segment (start 104.34 156.54) (end 104.5 156.7) (width 0.5) (layer "F.Cu") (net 2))
 (segment (start 92.5 156.54) (end 104.34 156.54) (width 0.5) (layer "F.Cu") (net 2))
 (segment (start 90.99 156.54) (end 92.5 156.54) (width 0.5) (layer "B.Cu") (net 2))
 (segment (start 89.73 155.28) (end 90.99 156.54) (width 0.5) (layer "B.Cu") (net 2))
 (segment (start 89.73 149.62) (end 89.73 155.28) (width 0.5) (layer "B.Cu") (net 2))
 (segment (start 82.59 146.73) (end 77.26 146.73) (width 0.5) (layer "F.Cu") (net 1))
 (segment (start 65 108.5) (end 58.85 108.5) (width 0.5) (layer "F.Cu") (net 1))
 (segment (start 58.85 108.5) (end 55.71 111.64) (width 0.5) (layer "F.Cu") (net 1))
 (segment (start 89.86 154) (end 82.59 146.73) (width 0.5) (layer "F.Cu") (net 1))
 (segment (start 101.2 147.08) (end 94.28 154) (width 0.5) (layer "F.Cu") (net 1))
 (segment (start 58.65 142.46) (end 71.35 142.46) (width 0.5) (layer "F.Cu") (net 1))
 (segment (start 55.71 111.64) (end 55.71 148.24) (width 0.5) (layer "F.Cu") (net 1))
 (segment (start 102.32 147.08) (end 101.2 147.08) (width 0.5) (layer "F.Cu") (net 1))
 (segment (start 94.28 154) (end 89.86 154) (width 0.5) (layer "F.Cu") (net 1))
 (segment (start 72.99 142.46) (end 71.35 142.46) (width 0.5) (layer "F.Cu") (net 1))
 (segment (start 55.71 148.24) (end 58.97 151.5) (width 0.5) (layer "F.Cu") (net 1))
 (segment (start 77.26 146.73) (end 72.99 142.46) (width 0.5) (layer "F.Cu") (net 1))
 (segment (start 58.97 151.5) (end 65 151.5) (width 0.5) (layer "F.Cu") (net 1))
 (segment (start 65 151.5) (end 65 143.31) (width 0.5) (layer "B.Cu") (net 1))
 (segment (start 65 143.31) (end 65.85 142.46) (width 0.5) (layer "B.Cu") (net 1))
 (segment (start 65.85 142.46) (end 71.35 142.46) (width 0.5) (layer "B.Cu") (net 1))
 (segment (start 125.65 147.54) (end 138.35 147.54) (width 0.5) (layer "F.Cu") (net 10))
 (segment (start 125.65 149.99) (end 121.48 154.16) (width 0.5) (layer "F.Cu") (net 10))
 (segment (start 121.48 154.16) (end 104.66 154.16) (width 0.5) (layer "F.Cu") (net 10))
 (segment (start 132 121.5) (end 132 138.5) (width 0.5) (layer "F.Cu") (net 10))
 (segment (start 125.65 147.54) (end 125.65 149.99) (width 0.5) (layer "F.Cu") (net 10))
 (segment (start 104.66 154.16) (end 104.5 154) (width 0.5) (layer "F.Cu") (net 10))
 (segment (start 132 146.68) (end 131.13 147.55) (width 0.5) (layer "B.Cu") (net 10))
 (segment (start 131.12 147.54) (end 125.65 147.54) (width 0.5) (layer "B.Cu") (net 10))
 (segment (start 131.13 147.55) (end 131.12 147.54) (width 0.5) (layer "B.Cu") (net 10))
 (segment (start 132 138.5) (end 132 146.68) (width 0.5) (layer "B.Cu") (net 10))
 (segment (start 103.19 144.54) (end 104.5 145.85) (width 0.5) (layer "B.Cu") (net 10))
 (segment (start 104.5 145.85) (end 104.5 154) (width 0.5) (layer "B.Cu") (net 10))
 (segment (start 102.32 144.54) (end 103.19 144.54) (width 0.5) (layer "B.Cu") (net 10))
 (segment (start 94.7 146.97) (end 94.7 147.08) (width 0.5) (layer "F.Cu") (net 3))
 (segment (start 138.35 112.46) (end 125.65 112.46) (width 0.5) (layer "F.Cu") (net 3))
 (segment (start 94.71 147.09) (end 94.7 147.08) (width 0.5) (layer "B.Cu") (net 3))
 (segment (start 119.66 136.54) (end 116.41 139.79) (width 0.5) (layer "B.Cu") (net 3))
 (segment (start 125.65 112.46) (end 124.44 112.46) (width 0.5) (layer "B.Cu") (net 3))
 (segment (start 99.2 145.21) (end 97.32 147.09) (width 0.5) (layer "B.Cu") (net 3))
 (segment (start 97.32 147.09) (end 94.71 147.09) (width 0.5) (layer "B.Cu") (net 3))
 (segment (start 101.25 139.79) (end 99.2 141.84) (width 0.5) (layer "B.Cu") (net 3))
 (segment (start 93.31 147.08) (end 94.7 147.08) (width 0.5) (layer "B.Cu") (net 3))
 (segment (start 119.66 117.24) (end 119.66 136.54) (width 0.5) (layer "B.Cu") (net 3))
 (segment (start 124.44 112.46) (end 119.66 117.24) (width 0.5) (layer "B.Cu") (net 3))
 (segment (start 89.73 143.5) (end 93.31 147.08) (width 0.5) (layer "B.Cu") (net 3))
 (segment (start 116.41 139.79) (end 101.25 139.79) (width 0.5) (layer "B.Cu") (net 3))
 (segment (start 99.2 141.84) (end 99.2 145.21) (width 0.5) (layer "B.Cu") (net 3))
 (segment (start 89.73 142) (end 89.73 143.5) (width 0.5) (layer "B.Cu") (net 3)))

